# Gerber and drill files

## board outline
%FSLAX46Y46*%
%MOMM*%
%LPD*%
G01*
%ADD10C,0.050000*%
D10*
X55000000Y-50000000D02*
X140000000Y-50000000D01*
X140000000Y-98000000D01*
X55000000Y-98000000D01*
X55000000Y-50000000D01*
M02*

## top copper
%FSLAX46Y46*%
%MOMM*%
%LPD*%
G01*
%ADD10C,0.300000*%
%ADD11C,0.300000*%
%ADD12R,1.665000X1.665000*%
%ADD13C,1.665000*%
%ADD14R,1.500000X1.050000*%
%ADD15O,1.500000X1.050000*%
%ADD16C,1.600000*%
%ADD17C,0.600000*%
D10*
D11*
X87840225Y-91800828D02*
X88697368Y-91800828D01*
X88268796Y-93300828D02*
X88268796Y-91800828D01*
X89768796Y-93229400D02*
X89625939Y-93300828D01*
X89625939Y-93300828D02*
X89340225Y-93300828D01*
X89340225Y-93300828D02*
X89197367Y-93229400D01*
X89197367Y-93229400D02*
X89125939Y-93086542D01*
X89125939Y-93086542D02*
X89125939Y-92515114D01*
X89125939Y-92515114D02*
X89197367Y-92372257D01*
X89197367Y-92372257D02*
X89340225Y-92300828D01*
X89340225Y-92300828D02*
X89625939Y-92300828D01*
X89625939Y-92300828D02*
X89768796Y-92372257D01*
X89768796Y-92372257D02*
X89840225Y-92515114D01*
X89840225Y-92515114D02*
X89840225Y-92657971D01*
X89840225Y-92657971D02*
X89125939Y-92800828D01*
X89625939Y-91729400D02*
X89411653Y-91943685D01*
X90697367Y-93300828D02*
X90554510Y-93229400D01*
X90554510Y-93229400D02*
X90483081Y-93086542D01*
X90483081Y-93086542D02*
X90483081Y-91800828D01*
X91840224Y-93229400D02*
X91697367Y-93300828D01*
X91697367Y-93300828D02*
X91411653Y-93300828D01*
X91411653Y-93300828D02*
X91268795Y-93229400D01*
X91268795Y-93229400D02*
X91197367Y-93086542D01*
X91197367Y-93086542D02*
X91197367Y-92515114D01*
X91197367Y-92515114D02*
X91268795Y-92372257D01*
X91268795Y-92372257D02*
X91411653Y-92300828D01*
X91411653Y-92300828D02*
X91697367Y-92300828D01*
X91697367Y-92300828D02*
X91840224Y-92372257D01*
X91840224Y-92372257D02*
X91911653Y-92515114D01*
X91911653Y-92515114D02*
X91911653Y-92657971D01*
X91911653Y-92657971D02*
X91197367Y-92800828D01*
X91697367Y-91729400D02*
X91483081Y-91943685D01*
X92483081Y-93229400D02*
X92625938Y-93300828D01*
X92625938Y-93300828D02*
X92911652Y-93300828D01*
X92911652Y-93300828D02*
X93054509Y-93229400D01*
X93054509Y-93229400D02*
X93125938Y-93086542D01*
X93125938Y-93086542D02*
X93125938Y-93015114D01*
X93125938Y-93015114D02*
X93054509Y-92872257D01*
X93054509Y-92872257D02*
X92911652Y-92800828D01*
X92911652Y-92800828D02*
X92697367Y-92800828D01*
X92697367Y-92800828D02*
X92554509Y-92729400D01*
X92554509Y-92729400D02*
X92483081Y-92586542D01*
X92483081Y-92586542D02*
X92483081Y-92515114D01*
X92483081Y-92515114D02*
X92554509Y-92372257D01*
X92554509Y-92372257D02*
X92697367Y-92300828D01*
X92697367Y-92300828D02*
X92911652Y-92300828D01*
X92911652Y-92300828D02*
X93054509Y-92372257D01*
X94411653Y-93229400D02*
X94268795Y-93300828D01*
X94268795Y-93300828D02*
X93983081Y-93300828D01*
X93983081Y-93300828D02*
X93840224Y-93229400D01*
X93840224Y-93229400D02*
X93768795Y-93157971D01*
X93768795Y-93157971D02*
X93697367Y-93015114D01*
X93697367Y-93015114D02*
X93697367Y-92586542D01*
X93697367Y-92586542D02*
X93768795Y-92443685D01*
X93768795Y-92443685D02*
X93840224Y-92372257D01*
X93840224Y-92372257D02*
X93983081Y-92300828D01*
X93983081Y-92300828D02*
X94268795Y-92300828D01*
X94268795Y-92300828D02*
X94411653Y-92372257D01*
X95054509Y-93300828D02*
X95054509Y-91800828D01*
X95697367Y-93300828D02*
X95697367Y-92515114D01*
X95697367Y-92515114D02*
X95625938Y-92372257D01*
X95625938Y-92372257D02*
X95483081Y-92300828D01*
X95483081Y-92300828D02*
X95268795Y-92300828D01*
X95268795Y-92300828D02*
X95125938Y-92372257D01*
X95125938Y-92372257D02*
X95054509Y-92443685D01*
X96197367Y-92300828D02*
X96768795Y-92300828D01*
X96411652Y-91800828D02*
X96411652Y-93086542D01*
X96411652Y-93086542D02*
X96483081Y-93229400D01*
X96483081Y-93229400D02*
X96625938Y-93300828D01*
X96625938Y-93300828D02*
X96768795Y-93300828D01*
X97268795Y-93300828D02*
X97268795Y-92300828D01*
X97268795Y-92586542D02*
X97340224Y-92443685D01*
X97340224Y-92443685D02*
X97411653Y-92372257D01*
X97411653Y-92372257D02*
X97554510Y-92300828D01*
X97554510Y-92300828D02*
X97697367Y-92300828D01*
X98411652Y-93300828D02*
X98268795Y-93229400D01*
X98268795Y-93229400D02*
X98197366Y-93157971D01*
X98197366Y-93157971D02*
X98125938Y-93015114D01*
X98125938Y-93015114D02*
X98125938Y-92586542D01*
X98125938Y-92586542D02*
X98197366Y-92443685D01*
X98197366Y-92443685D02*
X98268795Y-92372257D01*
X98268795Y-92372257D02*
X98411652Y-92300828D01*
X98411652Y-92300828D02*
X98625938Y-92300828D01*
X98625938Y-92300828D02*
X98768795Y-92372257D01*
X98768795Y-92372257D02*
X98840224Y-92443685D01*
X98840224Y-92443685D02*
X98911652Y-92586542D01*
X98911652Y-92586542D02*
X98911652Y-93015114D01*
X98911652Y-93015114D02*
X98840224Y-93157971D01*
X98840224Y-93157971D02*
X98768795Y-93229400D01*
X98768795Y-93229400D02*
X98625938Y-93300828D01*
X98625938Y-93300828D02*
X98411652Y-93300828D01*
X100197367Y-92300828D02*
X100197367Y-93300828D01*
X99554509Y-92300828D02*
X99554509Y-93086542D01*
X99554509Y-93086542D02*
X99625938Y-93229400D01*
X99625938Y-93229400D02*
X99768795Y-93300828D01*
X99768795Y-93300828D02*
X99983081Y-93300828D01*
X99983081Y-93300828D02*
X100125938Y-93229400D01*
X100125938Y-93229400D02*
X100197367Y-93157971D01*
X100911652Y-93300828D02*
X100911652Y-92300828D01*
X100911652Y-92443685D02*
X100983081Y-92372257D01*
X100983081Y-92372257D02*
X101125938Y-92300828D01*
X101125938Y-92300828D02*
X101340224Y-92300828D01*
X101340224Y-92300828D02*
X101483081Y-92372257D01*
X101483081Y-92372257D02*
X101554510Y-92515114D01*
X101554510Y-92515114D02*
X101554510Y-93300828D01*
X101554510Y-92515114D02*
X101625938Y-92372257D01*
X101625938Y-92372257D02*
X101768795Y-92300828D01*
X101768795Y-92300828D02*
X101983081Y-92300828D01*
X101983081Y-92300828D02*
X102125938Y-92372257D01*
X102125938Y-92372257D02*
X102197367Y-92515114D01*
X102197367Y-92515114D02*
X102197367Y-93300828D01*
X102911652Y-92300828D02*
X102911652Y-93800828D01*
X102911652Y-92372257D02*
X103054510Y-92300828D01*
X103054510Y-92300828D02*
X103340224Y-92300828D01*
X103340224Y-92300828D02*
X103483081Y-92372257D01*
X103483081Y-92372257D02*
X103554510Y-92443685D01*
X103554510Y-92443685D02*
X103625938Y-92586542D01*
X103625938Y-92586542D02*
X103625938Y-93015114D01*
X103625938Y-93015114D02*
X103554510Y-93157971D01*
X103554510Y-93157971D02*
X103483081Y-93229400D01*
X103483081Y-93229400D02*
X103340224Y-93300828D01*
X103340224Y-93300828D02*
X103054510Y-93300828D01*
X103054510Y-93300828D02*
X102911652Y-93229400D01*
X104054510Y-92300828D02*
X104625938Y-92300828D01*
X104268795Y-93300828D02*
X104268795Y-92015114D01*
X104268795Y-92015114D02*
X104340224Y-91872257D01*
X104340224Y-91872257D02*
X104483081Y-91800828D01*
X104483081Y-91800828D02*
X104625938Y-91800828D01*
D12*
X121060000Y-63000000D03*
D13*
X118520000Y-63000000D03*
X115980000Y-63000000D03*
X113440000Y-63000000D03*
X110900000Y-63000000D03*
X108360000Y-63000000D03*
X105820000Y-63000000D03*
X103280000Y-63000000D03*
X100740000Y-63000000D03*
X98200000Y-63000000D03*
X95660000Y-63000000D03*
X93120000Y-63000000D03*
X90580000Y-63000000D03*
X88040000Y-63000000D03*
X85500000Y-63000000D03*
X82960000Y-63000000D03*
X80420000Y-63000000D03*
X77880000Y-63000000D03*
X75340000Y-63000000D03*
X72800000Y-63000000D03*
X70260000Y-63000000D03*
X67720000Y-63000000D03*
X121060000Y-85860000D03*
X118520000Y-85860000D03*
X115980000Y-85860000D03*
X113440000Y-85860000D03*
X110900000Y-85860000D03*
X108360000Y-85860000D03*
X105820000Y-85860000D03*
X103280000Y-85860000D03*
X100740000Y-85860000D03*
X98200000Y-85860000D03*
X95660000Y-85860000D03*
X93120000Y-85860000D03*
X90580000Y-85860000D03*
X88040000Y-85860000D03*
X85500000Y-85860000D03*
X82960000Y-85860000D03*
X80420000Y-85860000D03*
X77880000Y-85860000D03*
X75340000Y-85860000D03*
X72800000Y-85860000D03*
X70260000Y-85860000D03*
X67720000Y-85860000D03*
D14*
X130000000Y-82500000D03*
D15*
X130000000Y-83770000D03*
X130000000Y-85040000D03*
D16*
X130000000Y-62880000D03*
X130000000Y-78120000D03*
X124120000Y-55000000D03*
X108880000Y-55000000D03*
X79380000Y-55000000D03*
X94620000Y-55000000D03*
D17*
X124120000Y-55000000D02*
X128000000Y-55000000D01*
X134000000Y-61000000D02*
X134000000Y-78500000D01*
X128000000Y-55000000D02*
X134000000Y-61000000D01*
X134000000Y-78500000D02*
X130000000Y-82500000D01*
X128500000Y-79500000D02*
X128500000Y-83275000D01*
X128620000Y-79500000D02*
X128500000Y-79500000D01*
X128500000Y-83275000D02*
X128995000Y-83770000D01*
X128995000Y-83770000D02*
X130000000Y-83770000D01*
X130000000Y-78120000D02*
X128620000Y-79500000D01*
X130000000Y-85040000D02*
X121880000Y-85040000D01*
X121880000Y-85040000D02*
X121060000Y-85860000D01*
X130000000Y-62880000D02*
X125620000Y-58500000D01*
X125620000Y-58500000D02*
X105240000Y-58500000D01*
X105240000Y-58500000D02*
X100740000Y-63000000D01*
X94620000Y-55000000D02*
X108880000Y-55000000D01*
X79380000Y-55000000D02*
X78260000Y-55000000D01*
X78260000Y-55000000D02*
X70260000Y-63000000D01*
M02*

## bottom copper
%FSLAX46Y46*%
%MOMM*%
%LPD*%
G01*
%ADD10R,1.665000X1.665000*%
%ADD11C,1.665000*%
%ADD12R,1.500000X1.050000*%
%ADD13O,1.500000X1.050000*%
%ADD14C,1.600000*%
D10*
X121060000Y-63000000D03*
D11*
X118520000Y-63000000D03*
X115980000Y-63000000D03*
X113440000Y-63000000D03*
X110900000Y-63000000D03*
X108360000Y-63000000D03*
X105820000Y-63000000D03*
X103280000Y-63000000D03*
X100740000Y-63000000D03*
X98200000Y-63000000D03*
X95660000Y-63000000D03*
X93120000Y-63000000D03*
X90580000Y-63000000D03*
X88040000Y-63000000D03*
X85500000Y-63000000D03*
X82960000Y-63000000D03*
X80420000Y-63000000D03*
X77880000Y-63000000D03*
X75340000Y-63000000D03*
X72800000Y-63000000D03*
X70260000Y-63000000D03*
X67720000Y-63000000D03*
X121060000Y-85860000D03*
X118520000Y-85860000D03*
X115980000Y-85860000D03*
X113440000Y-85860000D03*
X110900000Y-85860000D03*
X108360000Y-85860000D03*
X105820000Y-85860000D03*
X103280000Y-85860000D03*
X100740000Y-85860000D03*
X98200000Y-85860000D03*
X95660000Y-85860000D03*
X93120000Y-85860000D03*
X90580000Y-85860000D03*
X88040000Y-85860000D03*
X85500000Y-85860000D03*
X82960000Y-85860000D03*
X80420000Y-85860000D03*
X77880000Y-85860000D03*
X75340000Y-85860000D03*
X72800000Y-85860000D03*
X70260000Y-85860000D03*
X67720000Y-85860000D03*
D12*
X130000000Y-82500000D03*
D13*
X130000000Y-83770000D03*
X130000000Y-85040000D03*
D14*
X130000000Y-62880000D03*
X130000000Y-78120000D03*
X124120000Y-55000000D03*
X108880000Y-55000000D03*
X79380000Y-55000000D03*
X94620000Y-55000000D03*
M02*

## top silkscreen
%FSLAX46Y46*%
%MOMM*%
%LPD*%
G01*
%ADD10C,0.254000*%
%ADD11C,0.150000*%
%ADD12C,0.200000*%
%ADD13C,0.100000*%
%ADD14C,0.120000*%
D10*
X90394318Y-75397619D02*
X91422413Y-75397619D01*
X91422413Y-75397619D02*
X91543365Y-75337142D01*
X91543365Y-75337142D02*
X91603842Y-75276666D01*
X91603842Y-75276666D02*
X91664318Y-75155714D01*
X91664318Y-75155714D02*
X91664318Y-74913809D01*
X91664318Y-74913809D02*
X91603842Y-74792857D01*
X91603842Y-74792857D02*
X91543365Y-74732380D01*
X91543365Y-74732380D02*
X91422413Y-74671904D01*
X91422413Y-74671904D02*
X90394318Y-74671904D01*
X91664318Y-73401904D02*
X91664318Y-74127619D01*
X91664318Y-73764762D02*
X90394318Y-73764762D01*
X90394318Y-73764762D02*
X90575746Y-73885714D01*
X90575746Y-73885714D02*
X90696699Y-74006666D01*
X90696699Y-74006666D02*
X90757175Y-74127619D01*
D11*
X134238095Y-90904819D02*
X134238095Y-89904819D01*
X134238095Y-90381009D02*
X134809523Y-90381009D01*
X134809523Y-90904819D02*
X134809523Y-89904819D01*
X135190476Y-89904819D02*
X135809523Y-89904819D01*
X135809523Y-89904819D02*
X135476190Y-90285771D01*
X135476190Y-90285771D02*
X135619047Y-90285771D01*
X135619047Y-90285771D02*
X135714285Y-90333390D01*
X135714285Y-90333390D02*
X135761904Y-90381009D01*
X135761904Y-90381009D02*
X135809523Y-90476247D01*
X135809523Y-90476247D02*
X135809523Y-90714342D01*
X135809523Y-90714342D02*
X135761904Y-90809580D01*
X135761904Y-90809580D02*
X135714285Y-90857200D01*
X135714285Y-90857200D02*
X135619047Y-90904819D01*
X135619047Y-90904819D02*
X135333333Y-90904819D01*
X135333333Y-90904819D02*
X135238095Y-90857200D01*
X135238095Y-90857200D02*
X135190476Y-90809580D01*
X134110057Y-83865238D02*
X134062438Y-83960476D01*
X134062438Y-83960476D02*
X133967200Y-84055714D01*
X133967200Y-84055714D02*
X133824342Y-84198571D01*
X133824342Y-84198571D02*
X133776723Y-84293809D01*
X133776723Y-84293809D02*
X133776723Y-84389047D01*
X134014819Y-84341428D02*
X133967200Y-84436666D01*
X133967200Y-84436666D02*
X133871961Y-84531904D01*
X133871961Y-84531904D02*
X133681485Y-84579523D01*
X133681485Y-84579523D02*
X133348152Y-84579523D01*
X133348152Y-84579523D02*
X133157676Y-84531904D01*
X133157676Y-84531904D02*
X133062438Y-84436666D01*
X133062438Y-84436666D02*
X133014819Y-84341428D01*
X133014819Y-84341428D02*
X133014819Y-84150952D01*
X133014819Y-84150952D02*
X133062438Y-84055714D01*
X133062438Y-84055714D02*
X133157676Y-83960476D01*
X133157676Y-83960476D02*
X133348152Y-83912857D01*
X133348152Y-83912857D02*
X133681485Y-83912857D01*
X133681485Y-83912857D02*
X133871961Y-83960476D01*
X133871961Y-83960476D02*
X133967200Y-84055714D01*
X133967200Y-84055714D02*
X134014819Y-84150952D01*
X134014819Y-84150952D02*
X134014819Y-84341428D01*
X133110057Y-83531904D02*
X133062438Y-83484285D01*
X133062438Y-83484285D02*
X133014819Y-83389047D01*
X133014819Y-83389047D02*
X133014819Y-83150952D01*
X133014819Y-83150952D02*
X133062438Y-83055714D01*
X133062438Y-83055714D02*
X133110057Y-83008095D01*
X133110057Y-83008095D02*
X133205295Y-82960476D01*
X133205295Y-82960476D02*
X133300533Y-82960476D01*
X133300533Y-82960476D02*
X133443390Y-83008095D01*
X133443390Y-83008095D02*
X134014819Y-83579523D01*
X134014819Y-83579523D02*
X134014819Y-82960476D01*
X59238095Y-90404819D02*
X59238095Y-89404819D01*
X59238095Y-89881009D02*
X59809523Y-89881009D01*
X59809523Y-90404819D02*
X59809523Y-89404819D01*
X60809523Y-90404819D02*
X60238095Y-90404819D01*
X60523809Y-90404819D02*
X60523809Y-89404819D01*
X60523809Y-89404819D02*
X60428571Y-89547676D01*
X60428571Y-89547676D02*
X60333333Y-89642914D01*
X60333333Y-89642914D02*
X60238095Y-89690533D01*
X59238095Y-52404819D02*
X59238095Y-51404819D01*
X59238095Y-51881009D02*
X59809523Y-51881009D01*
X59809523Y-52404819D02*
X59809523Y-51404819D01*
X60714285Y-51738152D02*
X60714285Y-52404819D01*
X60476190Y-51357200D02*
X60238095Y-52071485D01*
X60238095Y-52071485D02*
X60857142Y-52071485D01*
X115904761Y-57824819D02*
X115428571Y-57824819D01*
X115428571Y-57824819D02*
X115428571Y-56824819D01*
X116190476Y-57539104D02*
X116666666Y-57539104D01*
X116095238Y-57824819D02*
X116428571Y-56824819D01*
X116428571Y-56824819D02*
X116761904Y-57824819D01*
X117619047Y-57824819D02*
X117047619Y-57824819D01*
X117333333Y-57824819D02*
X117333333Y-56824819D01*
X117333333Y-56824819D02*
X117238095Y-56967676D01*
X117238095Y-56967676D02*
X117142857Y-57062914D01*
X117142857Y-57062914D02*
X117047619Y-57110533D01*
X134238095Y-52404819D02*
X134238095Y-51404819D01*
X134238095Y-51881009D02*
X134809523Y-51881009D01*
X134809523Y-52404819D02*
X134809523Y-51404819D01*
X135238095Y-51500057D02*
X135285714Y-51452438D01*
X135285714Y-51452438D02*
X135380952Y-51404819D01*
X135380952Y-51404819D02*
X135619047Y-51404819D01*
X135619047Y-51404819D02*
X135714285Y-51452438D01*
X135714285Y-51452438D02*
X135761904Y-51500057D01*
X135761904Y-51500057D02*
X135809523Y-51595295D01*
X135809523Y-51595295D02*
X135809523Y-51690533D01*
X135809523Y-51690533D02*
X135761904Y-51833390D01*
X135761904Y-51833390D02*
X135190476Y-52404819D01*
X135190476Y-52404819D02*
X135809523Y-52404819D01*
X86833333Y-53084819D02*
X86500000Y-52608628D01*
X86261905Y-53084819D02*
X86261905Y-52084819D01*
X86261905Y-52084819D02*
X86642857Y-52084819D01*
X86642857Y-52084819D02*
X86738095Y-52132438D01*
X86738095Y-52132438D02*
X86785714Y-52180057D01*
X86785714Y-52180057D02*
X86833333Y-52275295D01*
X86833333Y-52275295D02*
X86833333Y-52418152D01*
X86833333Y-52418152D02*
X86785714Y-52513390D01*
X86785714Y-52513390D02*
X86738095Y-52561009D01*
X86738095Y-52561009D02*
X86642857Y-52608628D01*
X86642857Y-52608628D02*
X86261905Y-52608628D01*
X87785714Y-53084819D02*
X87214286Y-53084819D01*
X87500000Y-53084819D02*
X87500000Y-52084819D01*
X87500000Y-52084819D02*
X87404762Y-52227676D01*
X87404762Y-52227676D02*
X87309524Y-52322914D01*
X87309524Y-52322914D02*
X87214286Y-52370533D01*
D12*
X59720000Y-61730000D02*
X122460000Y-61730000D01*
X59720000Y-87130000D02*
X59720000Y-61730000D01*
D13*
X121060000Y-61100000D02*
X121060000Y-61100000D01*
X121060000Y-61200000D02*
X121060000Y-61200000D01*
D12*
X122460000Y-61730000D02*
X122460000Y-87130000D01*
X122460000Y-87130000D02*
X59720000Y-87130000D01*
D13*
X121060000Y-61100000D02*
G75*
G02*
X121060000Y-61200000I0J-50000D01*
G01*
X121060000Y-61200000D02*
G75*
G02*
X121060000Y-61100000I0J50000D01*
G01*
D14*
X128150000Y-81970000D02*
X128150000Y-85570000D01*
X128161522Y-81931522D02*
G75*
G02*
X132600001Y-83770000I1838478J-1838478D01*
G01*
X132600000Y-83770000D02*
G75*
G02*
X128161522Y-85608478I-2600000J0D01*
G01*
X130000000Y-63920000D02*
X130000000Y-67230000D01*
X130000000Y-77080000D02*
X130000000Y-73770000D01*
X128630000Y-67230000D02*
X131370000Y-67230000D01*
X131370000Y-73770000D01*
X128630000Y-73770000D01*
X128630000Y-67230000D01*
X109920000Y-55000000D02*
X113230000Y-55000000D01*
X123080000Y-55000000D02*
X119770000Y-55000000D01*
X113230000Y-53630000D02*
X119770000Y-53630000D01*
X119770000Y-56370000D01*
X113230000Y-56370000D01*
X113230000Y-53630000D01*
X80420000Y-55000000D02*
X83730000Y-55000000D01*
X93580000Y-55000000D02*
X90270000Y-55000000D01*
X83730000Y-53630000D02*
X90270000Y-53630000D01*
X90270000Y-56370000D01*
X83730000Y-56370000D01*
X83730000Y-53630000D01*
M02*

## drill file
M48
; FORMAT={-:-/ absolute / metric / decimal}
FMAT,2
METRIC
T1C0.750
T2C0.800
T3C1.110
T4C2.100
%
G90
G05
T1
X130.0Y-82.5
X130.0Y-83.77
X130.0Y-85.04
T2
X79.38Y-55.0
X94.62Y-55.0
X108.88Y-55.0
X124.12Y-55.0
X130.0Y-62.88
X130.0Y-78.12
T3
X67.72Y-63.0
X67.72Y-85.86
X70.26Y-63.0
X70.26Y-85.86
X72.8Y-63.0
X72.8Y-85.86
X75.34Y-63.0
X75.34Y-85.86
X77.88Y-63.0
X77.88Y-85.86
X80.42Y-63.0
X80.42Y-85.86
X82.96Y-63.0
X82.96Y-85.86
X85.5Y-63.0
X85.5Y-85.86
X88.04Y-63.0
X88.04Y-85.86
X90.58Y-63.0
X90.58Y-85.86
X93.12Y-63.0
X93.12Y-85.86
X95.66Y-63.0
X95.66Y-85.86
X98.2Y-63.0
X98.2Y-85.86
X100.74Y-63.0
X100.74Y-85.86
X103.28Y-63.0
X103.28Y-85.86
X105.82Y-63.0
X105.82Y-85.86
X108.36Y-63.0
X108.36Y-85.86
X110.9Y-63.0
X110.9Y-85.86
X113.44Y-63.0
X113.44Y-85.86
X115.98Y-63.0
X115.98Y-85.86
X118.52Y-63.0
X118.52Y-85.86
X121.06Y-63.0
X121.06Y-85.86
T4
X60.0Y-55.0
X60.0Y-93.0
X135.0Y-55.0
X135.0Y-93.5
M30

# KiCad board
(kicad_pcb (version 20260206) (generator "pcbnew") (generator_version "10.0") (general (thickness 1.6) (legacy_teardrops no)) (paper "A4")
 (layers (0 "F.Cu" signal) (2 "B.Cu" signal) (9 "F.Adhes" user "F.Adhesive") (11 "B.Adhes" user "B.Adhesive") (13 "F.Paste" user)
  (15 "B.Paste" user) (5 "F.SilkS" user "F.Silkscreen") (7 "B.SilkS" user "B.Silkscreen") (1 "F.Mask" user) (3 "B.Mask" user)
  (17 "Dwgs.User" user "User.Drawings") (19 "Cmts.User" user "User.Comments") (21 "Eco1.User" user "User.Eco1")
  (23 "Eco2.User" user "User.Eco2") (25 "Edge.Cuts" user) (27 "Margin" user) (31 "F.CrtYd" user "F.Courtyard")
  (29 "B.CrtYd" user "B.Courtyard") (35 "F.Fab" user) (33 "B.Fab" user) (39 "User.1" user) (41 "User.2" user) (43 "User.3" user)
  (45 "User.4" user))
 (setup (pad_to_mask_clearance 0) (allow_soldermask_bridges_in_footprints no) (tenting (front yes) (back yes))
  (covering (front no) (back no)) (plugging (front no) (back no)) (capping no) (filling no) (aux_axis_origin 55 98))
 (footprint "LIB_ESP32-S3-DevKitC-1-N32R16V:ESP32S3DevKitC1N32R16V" (layer "F.Cu") (at 121.06 63 -90)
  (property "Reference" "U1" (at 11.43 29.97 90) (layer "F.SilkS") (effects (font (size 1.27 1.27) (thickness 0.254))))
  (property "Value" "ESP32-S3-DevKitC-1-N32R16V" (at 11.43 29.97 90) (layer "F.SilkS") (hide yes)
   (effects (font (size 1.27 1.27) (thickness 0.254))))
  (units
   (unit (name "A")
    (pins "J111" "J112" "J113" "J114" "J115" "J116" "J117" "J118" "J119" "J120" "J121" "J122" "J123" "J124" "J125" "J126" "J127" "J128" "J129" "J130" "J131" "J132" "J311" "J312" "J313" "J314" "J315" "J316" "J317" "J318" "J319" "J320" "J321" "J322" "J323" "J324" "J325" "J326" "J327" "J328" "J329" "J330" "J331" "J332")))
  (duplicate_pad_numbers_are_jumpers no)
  (fp_line (start -1.27 61.34) (end -1.27 -1.4) (stroke (width 0.2) (type solid)) (layer "F.SilkS"))
  (fp_line (start 24.13 61.34) (end -1.27 61.34) (stroke (width 0.2) (type solid)) (layer "F.SilkS"))
  (fp_line (start -1.9 0) (end -1.9 0) (stroke (width 0.1) (type solid)) (layer "F.SilkS"))
  (fp_line (start -1.8 0) (end -1.8 0) (stroke (width 0.1) (type solid)) (layer "F.SilkS"))
  (fp_line (start -1.27 -1.4) (end 24.13 -1.4) (stroke (width 0.2) (type solid)) (layer "F.SilkS"))
  (fp_line (start 24.13 -1.4) (end 24.13 61.34) (stroke (width 0.2) (type solid)) (layer "F.SilkS"))
  (fp_arc (start -1.9 0) (mid -1.85 -0.05) (end -1.8 0) (stroke (width 0.1) (type solid)) (layer "F.SilkS"))
  (fp_arc (start -1.8 0) (mid -1.85 0.05) (end -1.9 0) (stroke (width 0.1) (type solid)) (layer "F.SilkS"))
  (pad "J111" thru_hole rect (at 0 0 270) (size 1.665 1.665) (drill 1.11) (layers "*.Cu" "*.Mask") (remove_unused_layers no)
   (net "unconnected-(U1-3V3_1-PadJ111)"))
  (pad "J112" thru_hole circle (at 0 2.54 270) (size 1.665 1.665) (drill 1.11) (layers "*.Cu" "*.Mask") (remove_unused_layers no)
   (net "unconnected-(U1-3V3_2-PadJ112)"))
  (pad "J113" thru_hole circle (at 0 5.08 270) (size 1.665 1.665) (drill 1.11) (layers "*.Cu" "*.Mask") (remove_unused_layers no)
   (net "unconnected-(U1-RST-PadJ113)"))
  (pad "J114" thru_hole circle (at 0 7.62 270) (size 1.665 1.665) (drill 1.11) (layers "*.Cu" "*.Mask") (remove_unused_layers no)
   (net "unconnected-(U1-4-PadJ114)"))
  (pad "J115" thru_hole circle (at 0 10.16 270) (size 1.665 1.665) (drill 1.11) (layers "*.Cu" "*.Mask") (remove_unused_layers no)
   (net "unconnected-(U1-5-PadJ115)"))
  (pad "J116" thru_hole circle (at 0 12.7 270) (size 1.665 1.665) (drill 1.11) (layers "*.Cu" "*.Mask") (remove_unused_layers no)
   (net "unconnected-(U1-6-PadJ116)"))
  (pad "J117" thru_hole circle (at 0 15.24 270) (size 1.665 1.665) (drill 1.11) (layers "*.Cu" "*.Mask") (remove_unused_layers no)
   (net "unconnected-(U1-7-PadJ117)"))
  (pad "J118" thru_hole circle (at 0 17.78 270) (size 1.665 1.665) (drill 1.11) (layers "*.Cu" "*.Mask") (remove_unused_layers no)
   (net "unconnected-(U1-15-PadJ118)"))
  (pad "J119" thru_hole circle (at 0 20.32 270) (size 1.665 1.665) (drill 1.11) (layers "*.Cu" "*.Mask") (remove_unused_layers no)
   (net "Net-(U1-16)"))
  (pad "J120" thru_hole circle (at 0 22.86 270) (size 1.665 1.665) (drill 1.11) (layers "*.Cu" "*.Mask") (remove_unused_layers no)
   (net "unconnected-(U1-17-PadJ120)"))
  (pad "J121" thru_hole circle (at 0 25.4 270) (size 1.665 1.665) (drill 1.11) (layers "*.Cu" "*.Mask") (remove_unused_layers no)
   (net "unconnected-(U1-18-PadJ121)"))
  (pad "J122" thru_hole circle (at 0 27.94 270) (size 1.665 1.665) (drill 1.11) (layers "*.Cu" "*.Mask") (remove_unused_layers no)
   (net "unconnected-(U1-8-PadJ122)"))
  (pad "J123" thru_hole circle (at 0 30.48 270) (size 1.665 1.665) (drill 1.11) (layers "*.Cu" "*.Mask") (remove_unused_layers no)
   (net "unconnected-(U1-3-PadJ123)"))
  (pad "J124" thru_hole circle (at 0 33.02 270) (size 1.665 1.665) (drill 1.11) (layers "*.Cu" "*.Mask") (remove_unused_layers no)
   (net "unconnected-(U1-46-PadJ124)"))
  (pad "J125" thru_hole circle (at 0 35.56 270) (size 1.665 1.665) (drill 1.11) (layers "*.Cu" "*.Mask") (remove_unused_layers no)
   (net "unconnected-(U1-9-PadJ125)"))
  (pad "J126" thru_hole circle (at 0 38.1 270) (size 1.665 1.665) (drill 1.11) (layers "*.Cu" "*.Mask") (remove_unused_layers no)
   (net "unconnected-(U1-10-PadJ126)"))
  (pad "J127" thru_hole circle (at 0 40.64 270) (size 1.665 1.665) (drill 1.11) (layers "*.Cu" "*.Mask") (remove_unused_layers no)
   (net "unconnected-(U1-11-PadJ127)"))
  (pad "J128" thru_hole circle (at 0 43.18 270) (size 1.665 1.665) (drill 1.11) (layers "*.Cu" "*.Mask") (remove_unused_layers no)
   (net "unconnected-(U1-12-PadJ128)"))
  (pad "J129" thru_hole circle (at 0 45.72 270) (size 1.665 1.665) (drill 1.11) (layers "*.Cu" "*.Mask") (remove_unused_layers no)
   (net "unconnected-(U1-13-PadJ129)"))
  (pad "J130" thru_hole circle (at 0 48.26 270) (size 1.665 1.665) (drill 1.11) (layers "*.Cu" "*.Mask") (remove_unused_layers no)
   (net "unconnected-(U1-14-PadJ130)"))
  (pad "J131" thru_hole circle (at 0 50.8 270) (size 1.665 1.665) (drill 1.11) (layers "*.Cu" "*.Mask") (remove_unused_layers no)
   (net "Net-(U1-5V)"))
  (pad "J132" thru_hole circle (at 0 53.34 270) (size 1.665 1.665) (drill 1.11) (layers "*.Cu" "*.Mask") (remove_unused_layers no)
   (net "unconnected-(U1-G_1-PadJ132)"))
  (pad "J311" thru_hole circle (at 22.86 0 270) (size 1.665 1.665) (drill 1.11) (layers "*.Cu" "*.Mask") (remove_unused_layers no)
   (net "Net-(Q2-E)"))
  (pad "J312" thru_hole circle (at 22.86 2.54 270) (size 1.665 1.665) (drill 1.11) (layers "*.Cu" "*.Mask") (remove_unused_layers no)
   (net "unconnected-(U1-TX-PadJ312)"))
  (pad "J313" thru_hole circle (at 22.86 5.08 270) (size 1.665 1.665) (drill 1.11) (layers "*.Cu" "*.Mask") (remove_unused_layers no)
   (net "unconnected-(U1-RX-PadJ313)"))
  (pad "J314" thru_hole circle (at 22.86 7.62 270) (size 1.665 1.665) (drill 1.11) (layers "*.Cu" "*.Mask") (remove_unused_layers no)
   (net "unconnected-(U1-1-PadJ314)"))
  (pad "J315" thru_hole circle (at 22.86 10.16 270) (size 1.665 1.665) (drill 1.11) (layers "*.Cu" "*.Mask") (remove_unused_layers no)
   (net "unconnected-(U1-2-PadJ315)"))
  (pad "J316" thru_hole circle (at 22.86 12.7 270) (size 1.665 1.665) (drill 1.11) (layers "*.Cu" "*.Mask") (remove_unused_layers no)
   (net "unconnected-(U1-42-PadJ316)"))
  (pad "J317" thru_hole circle (at 22.86 15.24 270) (size 1.665 1.665) (drill 1.11) (layers "*.Cu" "*.Mask") (remove_unused_layers no)
   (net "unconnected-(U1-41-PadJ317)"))
  (pad "J318" thru_hole circle (at 22.86 17.78 270) (size 1.665 1.665) (drill 1.11) (layers "*.Cu" "*.Mask") (remove_unused_layers no)
   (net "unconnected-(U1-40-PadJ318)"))
  (pad "J319" thru_hole circle (at 22.86 20.32 270) (size 1.665 1.665) (drill 1.11) (layers "*.Cu" "*.Mask") (remove_unused_layers no)
   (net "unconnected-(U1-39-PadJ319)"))
  (pad "J320" thru_hole circle (at 22.86 22.86 270) (size 1.665 1.665) (drill 1.11) (layers "*.Cu" "*.Mask") (remove_unused_layers no)
   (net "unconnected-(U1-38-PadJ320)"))
  (pad "J321" thru_hole circle (at 22.86 25.4 270) (size 1.665 1.665) (drill 1.11) (layers "*.Cu" "*.Mask") (remove_unused_layers no)
   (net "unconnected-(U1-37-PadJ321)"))
  (pad "J322" thru_hole circle (at 22.86 27.94 270) (size 1.665 1.665) (drill 1.11) (layers "*.Cu" "*.Mask") (remove_unused_layers no)
   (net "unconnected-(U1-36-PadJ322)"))
  (pad "J323" thru_hole circle (at 22.86 30.48 270) (size 1.665 1.665) (drill 1.11) (layers "*.Cu" "*.Mask") (remove_unused_layers no)
   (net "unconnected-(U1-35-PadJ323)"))
  (pad "J324" thru_hole circle (at 22.86 33.02 270) (size 1.665 1.665) (drill 1.11) (layers "*.Cu" "*.Mask") (remove_unused_layers no)
   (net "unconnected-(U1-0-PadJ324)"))
  (pad "J325" thru_hole circle (at 22.86 35.56 270) (size 1.665 1.665) (drill 1.11) (layers "*.Cu" "*.Mask") (remove_unused_layers no)
   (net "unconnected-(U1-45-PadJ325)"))
  (pad "J326" thru_hole circle (at 22.86 38.1 270) (size 1.665 1.665) (drill 1.11) (layers "*.Cu" "*.Mask") (remove_unused_layers no)
   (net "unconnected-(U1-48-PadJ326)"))
  (pad "J327" thru_hole circle (at 22.86 40.64 270) (size 1.665 1.665) (drill 1.11) (layers "*.Cu" "*.Mask") (remove_unused_layers no)
   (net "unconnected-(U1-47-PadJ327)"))
  (pad "J328" thru_hole circle (at 22.86 43.18 270) (size 1.665 1.665) (drill 1.11) (layers "*.Cu" "*.Mask") (remove_unused_layers no)
   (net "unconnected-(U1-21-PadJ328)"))
  (pad "J329" thru_hole circle (at 22.86 45.72 270) (size 1.665 1.665) (drill 1.11) (layers "*.Cu" "*.Mask") (remove_unused_layers no)
   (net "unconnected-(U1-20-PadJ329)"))
  (pad "J330" thru_hole circle (at 22.86 48.26 270) (size 1.665 1.665) (drill 1.11) (layers "*.Cu" "*.Mask") (remove_unused_layers no)
   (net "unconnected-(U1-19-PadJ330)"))
  (pad "J331" thru_hole circle (at 22.86 50.8 270) (size 1.665 1.665) (drill 1.11) (layers "*.Cu" "*.Mask") (remove_unused_layers no)
   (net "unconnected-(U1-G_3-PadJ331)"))
  (pad "J332" thru_hole circle (at 22.86 53.34 270) (size 1.665 1.665) (drill 1.11) (layers "*.Cu" "*.Mask") (remove_unused_layers no)
   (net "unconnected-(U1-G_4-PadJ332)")))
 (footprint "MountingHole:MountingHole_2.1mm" (layer "F.Cu") (at 135 93.5)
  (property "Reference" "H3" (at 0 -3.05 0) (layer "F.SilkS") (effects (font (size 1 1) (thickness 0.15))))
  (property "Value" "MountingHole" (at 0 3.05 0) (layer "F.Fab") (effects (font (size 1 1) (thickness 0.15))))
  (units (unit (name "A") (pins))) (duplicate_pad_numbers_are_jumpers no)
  (pad "" np_thru_hole circle (at 0 0) (size 2.1 2.1) (drill 2.1) (layers "*.Cu" "*.Mask")))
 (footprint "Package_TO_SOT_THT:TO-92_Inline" (layer "F.Cu") (at 130 82.5 -90)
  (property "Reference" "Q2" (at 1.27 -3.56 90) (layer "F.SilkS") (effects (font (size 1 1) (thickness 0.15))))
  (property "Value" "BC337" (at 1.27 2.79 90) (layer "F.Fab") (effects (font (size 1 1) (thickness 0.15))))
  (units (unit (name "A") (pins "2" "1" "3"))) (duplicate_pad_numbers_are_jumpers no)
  (fp_line (start -0.53 1.85) (end 3.07 1.85) (stroke (width 0.12) (type solid)) (layer "F.SilkS"))
  (fp_arc (start -0.568478 1.838478) (mid -1.132087 -0.994977) (end 1.27 -2.6) (stroke (width 0.12) (type solid)) (layer "F.SilkS"))
  (fp_arc (start 1.27 -2.6) (mid 3.672087 -0.994977) (end 3.108478 1.838478) (stroke (width 0.12) (type solid)) (layer "F.SilkS"))
  (pad "1" thru_hole rect (at 0 0 270) (size 1.05 1.5) (drill 0.75) (layers "*.Cu" "*.Mask") (remove_unused_layers no) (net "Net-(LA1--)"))
  (pad "2" thru_hole oval (at 1.27 0 270) (size 1.05 1.5) (drill 0.75) (layers "*.Cu" "*.Mask") (remove_unused_layers no) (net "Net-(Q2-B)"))
  (pad "3" thru_hole oval (at 2.54 0 270) (size 1.05 1.5) (drill 0.75) (layers "*.Cu" "*.Mask") (remove_unused_layers no) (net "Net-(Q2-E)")))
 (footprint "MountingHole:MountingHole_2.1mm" (layer "F.Cu") (at 60 93)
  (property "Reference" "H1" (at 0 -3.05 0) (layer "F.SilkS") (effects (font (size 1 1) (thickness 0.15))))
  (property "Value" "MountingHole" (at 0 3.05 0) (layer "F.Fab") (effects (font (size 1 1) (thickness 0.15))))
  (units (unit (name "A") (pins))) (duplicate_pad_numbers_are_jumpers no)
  (pad "" np_thru_hole circle (at 0 0) (size 2.1 2.1) (drill 2.1) (layers "*.Cu" "*.Mask")))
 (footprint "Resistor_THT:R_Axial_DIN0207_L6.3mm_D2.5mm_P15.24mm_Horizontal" (layer "F.Cu") (at 130 62.88 -90)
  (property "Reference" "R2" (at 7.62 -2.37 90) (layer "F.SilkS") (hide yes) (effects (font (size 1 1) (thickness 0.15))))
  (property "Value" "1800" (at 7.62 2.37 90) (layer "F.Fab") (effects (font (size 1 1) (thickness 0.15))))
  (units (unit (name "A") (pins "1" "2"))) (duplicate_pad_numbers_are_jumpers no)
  (fp_line (start 1.04 0) (end 4.35 0) (stroke (width 0.12) (type solid)) (layer "F.SilkS"))
  (fp_line (start 14.2 0) (end 10.89 0) (stroke (width 0.12) (type solid)) (layer "F.SilkS"))
  (fp_rect (start 4.35 -1.37) (end 10.89 1.37) (stroke (width 0.12) (type solid)) (fill no) (layer "F.SilkS"))
  (pad "1" thru_hole circle (at 0 0 270) (size 1.6 1.6) (drill 0.8) (layers "*.Cu" "*.Mask") (remove_unused_layers no) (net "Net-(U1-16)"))
  (pad "2" thru_hole circle (at 15.24 0 270) (size 1.6 1.6) (drill 0.8) (layers "*.Cu" "*.Mask") (remove_unused_layers no)
   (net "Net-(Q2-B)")))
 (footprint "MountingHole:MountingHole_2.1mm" (layer "F.Cu") (at 60 55)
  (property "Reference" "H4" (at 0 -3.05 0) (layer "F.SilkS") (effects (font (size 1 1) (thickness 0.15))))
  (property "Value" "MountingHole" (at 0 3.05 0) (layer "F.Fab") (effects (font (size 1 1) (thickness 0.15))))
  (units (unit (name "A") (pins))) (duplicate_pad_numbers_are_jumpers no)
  (pad "" np_thru_hole circle (at 0 0) (size 2.1 2.1) (drill 2.1) (layers "*.Cu" "*.Mask")))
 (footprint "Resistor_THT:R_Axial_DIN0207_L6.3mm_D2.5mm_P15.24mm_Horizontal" (layer "F.Cu") (at 124.12 55 180)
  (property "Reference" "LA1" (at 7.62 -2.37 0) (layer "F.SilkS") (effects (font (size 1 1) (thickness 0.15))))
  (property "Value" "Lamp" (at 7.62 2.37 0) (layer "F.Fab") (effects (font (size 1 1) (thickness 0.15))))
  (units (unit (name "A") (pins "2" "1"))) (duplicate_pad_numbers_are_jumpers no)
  (fp_line (start 14.2 0) (end 10.89 0) (stroke (width 0.12) (type solid)) (layer "F.SilkS"))
  (fp_line (start 1.04 0) (end 4.35 0) (stroke (width 0.12) (type solid)) (layer "F.SilkS"))
  (fp_rect (start 4.35 -1.37) (end 10.89 1.37) (stroke (width 0.12) (type solid)) (fill no) (layer "F.SilkS"))
  (pad "1" thru_hole circle (at 0 0 180) (size 1.6 1.6) (drill 0.8) (layers "*.Cu" "*.Mask") (remove_unused_layers no) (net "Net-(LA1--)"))
  (pad "2" thru_hole circle (at 15.24 0 180) (size 1.6 1.6) (drill 0.8) (layers "*.Cu" "*.Mask") (remove_unused_layers no)
   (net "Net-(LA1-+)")))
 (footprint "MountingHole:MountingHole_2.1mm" (layer "F.Cu") (at 135 55)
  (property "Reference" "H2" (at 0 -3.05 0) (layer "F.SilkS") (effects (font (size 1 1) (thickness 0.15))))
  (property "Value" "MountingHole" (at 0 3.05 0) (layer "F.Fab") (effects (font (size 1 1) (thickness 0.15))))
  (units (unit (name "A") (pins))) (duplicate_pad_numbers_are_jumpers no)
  (pad "" np_thru_hole circle (at 0 0) (size 2.1 2.1) (drill 2.1) (layers "*.Cu" "*.Mask")))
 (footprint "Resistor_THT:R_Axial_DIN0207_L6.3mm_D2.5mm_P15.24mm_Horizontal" (layer "F.Cu") (at 79.38 55)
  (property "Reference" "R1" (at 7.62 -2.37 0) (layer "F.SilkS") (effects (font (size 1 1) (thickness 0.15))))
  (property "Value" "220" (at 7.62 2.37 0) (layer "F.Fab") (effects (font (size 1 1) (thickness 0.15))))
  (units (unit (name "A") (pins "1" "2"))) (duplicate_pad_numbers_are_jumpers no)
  (fp_line (start 1.04 0) (end 4.35 0) (stroke (width 0.12) (type solid)) (layer "F.SilkS"))
  (fp_line (start 14.2 0) (end 10.89 0) (stroke (width 0.12) (type solid)) (layer "F.SilkS"))
  (fp_rect (start 4.35 -1.37) (end 10.89 1.37) (stroke (width 0.12) (type solid)) (fill no) (layer "F.SilkS"))
  (pad "1" thru_hole circle (at 0 0) (size 1.6 1.6) (drill 0.8) (layers "*.Cu" "*.Mask") (remove_unused_layers no) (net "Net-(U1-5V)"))
  (pad "2" thru_hole circle (at 15.24 0) (size 1.6 1.6) (drill 0.8) (layers "*.Cu" "*.Mask") (remove_unused_layers no) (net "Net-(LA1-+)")))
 (gr_rect (start 55 50) (end 140 98) (stroke (width 0.05) (type default)) (fill no) (layer "Edge.Cuts"))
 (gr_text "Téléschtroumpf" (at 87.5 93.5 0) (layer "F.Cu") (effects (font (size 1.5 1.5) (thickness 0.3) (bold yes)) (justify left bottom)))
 (segment (start 124.12 55) (end 128 55) (width 0.6) (layer "F.Cu") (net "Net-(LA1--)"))
 (segment (start 134 61) (end 134 78.5) (width 0.6) (layer "F.Cu") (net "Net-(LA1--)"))
 (segment (start 128 55) (end 134 61) (width 0.6) (layer "F.Cu") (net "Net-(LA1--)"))
 (segment (start 134 78.5) (end 130 82.5) (width 0.6) (layer "F.Cu") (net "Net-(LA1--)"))
 (segment (start 128.5 79.5) (end 128.5 83.275) (width 0.6) (layer "F.Cu") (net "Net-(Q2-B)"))
 (segment (start 128.62 79.5) (end 128.5 79.5) (width 0.6) (layer "F.Cu") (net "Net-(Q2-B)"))
 (segment (start 128.5 83.275) (end 128.995 83.77) (width 0.6) (layer "F.Cu") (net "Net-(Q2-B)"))
 (segment (start 128.995 83.77) (end 130 83.77) (width 0.6) (layer "F.Cu") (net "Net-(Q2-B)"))
 (segment (start 130 78.12) (end 128.62 79.5) (width 0.6) (layer "F.Cu") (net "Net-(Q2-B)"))
 (segment (start 130 85.04) (end 121.88 85.04) (width 0.6) (layer "F.Cu") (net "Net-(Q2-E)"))
 (segment (start 121.88 85.04) (end 121.06 85.86) (width 0.6) (layer "F.Cu") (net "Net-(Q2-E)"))
 (segment (start 130 62.88) (end 125.62 58.5) (width 0.6) (layer "F.Cu") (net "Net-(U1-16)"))
 (segment (start 125.62 58.5) (end 105.24 58.5) (width 0.6) (layer "F.Cu") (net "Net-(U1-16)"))
 (segment (start 105.24 58.5) (end 100.74 63) (width 0.6) (layer "F.Cu") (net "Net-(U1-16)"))
 (segment (start 94.62 55) (end 108.88 55) (width 0.6) (layer "F.Cu") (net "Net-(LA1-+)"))
 (segment (start 79.38 55) (end 78.26 55) (width 0.6) (layer "F.Cu") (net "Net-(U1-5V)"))
 (segment (start 78.26 55) (end 70.26 63) (width 0.6) (layer "F.Cu") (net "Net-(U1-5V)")))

